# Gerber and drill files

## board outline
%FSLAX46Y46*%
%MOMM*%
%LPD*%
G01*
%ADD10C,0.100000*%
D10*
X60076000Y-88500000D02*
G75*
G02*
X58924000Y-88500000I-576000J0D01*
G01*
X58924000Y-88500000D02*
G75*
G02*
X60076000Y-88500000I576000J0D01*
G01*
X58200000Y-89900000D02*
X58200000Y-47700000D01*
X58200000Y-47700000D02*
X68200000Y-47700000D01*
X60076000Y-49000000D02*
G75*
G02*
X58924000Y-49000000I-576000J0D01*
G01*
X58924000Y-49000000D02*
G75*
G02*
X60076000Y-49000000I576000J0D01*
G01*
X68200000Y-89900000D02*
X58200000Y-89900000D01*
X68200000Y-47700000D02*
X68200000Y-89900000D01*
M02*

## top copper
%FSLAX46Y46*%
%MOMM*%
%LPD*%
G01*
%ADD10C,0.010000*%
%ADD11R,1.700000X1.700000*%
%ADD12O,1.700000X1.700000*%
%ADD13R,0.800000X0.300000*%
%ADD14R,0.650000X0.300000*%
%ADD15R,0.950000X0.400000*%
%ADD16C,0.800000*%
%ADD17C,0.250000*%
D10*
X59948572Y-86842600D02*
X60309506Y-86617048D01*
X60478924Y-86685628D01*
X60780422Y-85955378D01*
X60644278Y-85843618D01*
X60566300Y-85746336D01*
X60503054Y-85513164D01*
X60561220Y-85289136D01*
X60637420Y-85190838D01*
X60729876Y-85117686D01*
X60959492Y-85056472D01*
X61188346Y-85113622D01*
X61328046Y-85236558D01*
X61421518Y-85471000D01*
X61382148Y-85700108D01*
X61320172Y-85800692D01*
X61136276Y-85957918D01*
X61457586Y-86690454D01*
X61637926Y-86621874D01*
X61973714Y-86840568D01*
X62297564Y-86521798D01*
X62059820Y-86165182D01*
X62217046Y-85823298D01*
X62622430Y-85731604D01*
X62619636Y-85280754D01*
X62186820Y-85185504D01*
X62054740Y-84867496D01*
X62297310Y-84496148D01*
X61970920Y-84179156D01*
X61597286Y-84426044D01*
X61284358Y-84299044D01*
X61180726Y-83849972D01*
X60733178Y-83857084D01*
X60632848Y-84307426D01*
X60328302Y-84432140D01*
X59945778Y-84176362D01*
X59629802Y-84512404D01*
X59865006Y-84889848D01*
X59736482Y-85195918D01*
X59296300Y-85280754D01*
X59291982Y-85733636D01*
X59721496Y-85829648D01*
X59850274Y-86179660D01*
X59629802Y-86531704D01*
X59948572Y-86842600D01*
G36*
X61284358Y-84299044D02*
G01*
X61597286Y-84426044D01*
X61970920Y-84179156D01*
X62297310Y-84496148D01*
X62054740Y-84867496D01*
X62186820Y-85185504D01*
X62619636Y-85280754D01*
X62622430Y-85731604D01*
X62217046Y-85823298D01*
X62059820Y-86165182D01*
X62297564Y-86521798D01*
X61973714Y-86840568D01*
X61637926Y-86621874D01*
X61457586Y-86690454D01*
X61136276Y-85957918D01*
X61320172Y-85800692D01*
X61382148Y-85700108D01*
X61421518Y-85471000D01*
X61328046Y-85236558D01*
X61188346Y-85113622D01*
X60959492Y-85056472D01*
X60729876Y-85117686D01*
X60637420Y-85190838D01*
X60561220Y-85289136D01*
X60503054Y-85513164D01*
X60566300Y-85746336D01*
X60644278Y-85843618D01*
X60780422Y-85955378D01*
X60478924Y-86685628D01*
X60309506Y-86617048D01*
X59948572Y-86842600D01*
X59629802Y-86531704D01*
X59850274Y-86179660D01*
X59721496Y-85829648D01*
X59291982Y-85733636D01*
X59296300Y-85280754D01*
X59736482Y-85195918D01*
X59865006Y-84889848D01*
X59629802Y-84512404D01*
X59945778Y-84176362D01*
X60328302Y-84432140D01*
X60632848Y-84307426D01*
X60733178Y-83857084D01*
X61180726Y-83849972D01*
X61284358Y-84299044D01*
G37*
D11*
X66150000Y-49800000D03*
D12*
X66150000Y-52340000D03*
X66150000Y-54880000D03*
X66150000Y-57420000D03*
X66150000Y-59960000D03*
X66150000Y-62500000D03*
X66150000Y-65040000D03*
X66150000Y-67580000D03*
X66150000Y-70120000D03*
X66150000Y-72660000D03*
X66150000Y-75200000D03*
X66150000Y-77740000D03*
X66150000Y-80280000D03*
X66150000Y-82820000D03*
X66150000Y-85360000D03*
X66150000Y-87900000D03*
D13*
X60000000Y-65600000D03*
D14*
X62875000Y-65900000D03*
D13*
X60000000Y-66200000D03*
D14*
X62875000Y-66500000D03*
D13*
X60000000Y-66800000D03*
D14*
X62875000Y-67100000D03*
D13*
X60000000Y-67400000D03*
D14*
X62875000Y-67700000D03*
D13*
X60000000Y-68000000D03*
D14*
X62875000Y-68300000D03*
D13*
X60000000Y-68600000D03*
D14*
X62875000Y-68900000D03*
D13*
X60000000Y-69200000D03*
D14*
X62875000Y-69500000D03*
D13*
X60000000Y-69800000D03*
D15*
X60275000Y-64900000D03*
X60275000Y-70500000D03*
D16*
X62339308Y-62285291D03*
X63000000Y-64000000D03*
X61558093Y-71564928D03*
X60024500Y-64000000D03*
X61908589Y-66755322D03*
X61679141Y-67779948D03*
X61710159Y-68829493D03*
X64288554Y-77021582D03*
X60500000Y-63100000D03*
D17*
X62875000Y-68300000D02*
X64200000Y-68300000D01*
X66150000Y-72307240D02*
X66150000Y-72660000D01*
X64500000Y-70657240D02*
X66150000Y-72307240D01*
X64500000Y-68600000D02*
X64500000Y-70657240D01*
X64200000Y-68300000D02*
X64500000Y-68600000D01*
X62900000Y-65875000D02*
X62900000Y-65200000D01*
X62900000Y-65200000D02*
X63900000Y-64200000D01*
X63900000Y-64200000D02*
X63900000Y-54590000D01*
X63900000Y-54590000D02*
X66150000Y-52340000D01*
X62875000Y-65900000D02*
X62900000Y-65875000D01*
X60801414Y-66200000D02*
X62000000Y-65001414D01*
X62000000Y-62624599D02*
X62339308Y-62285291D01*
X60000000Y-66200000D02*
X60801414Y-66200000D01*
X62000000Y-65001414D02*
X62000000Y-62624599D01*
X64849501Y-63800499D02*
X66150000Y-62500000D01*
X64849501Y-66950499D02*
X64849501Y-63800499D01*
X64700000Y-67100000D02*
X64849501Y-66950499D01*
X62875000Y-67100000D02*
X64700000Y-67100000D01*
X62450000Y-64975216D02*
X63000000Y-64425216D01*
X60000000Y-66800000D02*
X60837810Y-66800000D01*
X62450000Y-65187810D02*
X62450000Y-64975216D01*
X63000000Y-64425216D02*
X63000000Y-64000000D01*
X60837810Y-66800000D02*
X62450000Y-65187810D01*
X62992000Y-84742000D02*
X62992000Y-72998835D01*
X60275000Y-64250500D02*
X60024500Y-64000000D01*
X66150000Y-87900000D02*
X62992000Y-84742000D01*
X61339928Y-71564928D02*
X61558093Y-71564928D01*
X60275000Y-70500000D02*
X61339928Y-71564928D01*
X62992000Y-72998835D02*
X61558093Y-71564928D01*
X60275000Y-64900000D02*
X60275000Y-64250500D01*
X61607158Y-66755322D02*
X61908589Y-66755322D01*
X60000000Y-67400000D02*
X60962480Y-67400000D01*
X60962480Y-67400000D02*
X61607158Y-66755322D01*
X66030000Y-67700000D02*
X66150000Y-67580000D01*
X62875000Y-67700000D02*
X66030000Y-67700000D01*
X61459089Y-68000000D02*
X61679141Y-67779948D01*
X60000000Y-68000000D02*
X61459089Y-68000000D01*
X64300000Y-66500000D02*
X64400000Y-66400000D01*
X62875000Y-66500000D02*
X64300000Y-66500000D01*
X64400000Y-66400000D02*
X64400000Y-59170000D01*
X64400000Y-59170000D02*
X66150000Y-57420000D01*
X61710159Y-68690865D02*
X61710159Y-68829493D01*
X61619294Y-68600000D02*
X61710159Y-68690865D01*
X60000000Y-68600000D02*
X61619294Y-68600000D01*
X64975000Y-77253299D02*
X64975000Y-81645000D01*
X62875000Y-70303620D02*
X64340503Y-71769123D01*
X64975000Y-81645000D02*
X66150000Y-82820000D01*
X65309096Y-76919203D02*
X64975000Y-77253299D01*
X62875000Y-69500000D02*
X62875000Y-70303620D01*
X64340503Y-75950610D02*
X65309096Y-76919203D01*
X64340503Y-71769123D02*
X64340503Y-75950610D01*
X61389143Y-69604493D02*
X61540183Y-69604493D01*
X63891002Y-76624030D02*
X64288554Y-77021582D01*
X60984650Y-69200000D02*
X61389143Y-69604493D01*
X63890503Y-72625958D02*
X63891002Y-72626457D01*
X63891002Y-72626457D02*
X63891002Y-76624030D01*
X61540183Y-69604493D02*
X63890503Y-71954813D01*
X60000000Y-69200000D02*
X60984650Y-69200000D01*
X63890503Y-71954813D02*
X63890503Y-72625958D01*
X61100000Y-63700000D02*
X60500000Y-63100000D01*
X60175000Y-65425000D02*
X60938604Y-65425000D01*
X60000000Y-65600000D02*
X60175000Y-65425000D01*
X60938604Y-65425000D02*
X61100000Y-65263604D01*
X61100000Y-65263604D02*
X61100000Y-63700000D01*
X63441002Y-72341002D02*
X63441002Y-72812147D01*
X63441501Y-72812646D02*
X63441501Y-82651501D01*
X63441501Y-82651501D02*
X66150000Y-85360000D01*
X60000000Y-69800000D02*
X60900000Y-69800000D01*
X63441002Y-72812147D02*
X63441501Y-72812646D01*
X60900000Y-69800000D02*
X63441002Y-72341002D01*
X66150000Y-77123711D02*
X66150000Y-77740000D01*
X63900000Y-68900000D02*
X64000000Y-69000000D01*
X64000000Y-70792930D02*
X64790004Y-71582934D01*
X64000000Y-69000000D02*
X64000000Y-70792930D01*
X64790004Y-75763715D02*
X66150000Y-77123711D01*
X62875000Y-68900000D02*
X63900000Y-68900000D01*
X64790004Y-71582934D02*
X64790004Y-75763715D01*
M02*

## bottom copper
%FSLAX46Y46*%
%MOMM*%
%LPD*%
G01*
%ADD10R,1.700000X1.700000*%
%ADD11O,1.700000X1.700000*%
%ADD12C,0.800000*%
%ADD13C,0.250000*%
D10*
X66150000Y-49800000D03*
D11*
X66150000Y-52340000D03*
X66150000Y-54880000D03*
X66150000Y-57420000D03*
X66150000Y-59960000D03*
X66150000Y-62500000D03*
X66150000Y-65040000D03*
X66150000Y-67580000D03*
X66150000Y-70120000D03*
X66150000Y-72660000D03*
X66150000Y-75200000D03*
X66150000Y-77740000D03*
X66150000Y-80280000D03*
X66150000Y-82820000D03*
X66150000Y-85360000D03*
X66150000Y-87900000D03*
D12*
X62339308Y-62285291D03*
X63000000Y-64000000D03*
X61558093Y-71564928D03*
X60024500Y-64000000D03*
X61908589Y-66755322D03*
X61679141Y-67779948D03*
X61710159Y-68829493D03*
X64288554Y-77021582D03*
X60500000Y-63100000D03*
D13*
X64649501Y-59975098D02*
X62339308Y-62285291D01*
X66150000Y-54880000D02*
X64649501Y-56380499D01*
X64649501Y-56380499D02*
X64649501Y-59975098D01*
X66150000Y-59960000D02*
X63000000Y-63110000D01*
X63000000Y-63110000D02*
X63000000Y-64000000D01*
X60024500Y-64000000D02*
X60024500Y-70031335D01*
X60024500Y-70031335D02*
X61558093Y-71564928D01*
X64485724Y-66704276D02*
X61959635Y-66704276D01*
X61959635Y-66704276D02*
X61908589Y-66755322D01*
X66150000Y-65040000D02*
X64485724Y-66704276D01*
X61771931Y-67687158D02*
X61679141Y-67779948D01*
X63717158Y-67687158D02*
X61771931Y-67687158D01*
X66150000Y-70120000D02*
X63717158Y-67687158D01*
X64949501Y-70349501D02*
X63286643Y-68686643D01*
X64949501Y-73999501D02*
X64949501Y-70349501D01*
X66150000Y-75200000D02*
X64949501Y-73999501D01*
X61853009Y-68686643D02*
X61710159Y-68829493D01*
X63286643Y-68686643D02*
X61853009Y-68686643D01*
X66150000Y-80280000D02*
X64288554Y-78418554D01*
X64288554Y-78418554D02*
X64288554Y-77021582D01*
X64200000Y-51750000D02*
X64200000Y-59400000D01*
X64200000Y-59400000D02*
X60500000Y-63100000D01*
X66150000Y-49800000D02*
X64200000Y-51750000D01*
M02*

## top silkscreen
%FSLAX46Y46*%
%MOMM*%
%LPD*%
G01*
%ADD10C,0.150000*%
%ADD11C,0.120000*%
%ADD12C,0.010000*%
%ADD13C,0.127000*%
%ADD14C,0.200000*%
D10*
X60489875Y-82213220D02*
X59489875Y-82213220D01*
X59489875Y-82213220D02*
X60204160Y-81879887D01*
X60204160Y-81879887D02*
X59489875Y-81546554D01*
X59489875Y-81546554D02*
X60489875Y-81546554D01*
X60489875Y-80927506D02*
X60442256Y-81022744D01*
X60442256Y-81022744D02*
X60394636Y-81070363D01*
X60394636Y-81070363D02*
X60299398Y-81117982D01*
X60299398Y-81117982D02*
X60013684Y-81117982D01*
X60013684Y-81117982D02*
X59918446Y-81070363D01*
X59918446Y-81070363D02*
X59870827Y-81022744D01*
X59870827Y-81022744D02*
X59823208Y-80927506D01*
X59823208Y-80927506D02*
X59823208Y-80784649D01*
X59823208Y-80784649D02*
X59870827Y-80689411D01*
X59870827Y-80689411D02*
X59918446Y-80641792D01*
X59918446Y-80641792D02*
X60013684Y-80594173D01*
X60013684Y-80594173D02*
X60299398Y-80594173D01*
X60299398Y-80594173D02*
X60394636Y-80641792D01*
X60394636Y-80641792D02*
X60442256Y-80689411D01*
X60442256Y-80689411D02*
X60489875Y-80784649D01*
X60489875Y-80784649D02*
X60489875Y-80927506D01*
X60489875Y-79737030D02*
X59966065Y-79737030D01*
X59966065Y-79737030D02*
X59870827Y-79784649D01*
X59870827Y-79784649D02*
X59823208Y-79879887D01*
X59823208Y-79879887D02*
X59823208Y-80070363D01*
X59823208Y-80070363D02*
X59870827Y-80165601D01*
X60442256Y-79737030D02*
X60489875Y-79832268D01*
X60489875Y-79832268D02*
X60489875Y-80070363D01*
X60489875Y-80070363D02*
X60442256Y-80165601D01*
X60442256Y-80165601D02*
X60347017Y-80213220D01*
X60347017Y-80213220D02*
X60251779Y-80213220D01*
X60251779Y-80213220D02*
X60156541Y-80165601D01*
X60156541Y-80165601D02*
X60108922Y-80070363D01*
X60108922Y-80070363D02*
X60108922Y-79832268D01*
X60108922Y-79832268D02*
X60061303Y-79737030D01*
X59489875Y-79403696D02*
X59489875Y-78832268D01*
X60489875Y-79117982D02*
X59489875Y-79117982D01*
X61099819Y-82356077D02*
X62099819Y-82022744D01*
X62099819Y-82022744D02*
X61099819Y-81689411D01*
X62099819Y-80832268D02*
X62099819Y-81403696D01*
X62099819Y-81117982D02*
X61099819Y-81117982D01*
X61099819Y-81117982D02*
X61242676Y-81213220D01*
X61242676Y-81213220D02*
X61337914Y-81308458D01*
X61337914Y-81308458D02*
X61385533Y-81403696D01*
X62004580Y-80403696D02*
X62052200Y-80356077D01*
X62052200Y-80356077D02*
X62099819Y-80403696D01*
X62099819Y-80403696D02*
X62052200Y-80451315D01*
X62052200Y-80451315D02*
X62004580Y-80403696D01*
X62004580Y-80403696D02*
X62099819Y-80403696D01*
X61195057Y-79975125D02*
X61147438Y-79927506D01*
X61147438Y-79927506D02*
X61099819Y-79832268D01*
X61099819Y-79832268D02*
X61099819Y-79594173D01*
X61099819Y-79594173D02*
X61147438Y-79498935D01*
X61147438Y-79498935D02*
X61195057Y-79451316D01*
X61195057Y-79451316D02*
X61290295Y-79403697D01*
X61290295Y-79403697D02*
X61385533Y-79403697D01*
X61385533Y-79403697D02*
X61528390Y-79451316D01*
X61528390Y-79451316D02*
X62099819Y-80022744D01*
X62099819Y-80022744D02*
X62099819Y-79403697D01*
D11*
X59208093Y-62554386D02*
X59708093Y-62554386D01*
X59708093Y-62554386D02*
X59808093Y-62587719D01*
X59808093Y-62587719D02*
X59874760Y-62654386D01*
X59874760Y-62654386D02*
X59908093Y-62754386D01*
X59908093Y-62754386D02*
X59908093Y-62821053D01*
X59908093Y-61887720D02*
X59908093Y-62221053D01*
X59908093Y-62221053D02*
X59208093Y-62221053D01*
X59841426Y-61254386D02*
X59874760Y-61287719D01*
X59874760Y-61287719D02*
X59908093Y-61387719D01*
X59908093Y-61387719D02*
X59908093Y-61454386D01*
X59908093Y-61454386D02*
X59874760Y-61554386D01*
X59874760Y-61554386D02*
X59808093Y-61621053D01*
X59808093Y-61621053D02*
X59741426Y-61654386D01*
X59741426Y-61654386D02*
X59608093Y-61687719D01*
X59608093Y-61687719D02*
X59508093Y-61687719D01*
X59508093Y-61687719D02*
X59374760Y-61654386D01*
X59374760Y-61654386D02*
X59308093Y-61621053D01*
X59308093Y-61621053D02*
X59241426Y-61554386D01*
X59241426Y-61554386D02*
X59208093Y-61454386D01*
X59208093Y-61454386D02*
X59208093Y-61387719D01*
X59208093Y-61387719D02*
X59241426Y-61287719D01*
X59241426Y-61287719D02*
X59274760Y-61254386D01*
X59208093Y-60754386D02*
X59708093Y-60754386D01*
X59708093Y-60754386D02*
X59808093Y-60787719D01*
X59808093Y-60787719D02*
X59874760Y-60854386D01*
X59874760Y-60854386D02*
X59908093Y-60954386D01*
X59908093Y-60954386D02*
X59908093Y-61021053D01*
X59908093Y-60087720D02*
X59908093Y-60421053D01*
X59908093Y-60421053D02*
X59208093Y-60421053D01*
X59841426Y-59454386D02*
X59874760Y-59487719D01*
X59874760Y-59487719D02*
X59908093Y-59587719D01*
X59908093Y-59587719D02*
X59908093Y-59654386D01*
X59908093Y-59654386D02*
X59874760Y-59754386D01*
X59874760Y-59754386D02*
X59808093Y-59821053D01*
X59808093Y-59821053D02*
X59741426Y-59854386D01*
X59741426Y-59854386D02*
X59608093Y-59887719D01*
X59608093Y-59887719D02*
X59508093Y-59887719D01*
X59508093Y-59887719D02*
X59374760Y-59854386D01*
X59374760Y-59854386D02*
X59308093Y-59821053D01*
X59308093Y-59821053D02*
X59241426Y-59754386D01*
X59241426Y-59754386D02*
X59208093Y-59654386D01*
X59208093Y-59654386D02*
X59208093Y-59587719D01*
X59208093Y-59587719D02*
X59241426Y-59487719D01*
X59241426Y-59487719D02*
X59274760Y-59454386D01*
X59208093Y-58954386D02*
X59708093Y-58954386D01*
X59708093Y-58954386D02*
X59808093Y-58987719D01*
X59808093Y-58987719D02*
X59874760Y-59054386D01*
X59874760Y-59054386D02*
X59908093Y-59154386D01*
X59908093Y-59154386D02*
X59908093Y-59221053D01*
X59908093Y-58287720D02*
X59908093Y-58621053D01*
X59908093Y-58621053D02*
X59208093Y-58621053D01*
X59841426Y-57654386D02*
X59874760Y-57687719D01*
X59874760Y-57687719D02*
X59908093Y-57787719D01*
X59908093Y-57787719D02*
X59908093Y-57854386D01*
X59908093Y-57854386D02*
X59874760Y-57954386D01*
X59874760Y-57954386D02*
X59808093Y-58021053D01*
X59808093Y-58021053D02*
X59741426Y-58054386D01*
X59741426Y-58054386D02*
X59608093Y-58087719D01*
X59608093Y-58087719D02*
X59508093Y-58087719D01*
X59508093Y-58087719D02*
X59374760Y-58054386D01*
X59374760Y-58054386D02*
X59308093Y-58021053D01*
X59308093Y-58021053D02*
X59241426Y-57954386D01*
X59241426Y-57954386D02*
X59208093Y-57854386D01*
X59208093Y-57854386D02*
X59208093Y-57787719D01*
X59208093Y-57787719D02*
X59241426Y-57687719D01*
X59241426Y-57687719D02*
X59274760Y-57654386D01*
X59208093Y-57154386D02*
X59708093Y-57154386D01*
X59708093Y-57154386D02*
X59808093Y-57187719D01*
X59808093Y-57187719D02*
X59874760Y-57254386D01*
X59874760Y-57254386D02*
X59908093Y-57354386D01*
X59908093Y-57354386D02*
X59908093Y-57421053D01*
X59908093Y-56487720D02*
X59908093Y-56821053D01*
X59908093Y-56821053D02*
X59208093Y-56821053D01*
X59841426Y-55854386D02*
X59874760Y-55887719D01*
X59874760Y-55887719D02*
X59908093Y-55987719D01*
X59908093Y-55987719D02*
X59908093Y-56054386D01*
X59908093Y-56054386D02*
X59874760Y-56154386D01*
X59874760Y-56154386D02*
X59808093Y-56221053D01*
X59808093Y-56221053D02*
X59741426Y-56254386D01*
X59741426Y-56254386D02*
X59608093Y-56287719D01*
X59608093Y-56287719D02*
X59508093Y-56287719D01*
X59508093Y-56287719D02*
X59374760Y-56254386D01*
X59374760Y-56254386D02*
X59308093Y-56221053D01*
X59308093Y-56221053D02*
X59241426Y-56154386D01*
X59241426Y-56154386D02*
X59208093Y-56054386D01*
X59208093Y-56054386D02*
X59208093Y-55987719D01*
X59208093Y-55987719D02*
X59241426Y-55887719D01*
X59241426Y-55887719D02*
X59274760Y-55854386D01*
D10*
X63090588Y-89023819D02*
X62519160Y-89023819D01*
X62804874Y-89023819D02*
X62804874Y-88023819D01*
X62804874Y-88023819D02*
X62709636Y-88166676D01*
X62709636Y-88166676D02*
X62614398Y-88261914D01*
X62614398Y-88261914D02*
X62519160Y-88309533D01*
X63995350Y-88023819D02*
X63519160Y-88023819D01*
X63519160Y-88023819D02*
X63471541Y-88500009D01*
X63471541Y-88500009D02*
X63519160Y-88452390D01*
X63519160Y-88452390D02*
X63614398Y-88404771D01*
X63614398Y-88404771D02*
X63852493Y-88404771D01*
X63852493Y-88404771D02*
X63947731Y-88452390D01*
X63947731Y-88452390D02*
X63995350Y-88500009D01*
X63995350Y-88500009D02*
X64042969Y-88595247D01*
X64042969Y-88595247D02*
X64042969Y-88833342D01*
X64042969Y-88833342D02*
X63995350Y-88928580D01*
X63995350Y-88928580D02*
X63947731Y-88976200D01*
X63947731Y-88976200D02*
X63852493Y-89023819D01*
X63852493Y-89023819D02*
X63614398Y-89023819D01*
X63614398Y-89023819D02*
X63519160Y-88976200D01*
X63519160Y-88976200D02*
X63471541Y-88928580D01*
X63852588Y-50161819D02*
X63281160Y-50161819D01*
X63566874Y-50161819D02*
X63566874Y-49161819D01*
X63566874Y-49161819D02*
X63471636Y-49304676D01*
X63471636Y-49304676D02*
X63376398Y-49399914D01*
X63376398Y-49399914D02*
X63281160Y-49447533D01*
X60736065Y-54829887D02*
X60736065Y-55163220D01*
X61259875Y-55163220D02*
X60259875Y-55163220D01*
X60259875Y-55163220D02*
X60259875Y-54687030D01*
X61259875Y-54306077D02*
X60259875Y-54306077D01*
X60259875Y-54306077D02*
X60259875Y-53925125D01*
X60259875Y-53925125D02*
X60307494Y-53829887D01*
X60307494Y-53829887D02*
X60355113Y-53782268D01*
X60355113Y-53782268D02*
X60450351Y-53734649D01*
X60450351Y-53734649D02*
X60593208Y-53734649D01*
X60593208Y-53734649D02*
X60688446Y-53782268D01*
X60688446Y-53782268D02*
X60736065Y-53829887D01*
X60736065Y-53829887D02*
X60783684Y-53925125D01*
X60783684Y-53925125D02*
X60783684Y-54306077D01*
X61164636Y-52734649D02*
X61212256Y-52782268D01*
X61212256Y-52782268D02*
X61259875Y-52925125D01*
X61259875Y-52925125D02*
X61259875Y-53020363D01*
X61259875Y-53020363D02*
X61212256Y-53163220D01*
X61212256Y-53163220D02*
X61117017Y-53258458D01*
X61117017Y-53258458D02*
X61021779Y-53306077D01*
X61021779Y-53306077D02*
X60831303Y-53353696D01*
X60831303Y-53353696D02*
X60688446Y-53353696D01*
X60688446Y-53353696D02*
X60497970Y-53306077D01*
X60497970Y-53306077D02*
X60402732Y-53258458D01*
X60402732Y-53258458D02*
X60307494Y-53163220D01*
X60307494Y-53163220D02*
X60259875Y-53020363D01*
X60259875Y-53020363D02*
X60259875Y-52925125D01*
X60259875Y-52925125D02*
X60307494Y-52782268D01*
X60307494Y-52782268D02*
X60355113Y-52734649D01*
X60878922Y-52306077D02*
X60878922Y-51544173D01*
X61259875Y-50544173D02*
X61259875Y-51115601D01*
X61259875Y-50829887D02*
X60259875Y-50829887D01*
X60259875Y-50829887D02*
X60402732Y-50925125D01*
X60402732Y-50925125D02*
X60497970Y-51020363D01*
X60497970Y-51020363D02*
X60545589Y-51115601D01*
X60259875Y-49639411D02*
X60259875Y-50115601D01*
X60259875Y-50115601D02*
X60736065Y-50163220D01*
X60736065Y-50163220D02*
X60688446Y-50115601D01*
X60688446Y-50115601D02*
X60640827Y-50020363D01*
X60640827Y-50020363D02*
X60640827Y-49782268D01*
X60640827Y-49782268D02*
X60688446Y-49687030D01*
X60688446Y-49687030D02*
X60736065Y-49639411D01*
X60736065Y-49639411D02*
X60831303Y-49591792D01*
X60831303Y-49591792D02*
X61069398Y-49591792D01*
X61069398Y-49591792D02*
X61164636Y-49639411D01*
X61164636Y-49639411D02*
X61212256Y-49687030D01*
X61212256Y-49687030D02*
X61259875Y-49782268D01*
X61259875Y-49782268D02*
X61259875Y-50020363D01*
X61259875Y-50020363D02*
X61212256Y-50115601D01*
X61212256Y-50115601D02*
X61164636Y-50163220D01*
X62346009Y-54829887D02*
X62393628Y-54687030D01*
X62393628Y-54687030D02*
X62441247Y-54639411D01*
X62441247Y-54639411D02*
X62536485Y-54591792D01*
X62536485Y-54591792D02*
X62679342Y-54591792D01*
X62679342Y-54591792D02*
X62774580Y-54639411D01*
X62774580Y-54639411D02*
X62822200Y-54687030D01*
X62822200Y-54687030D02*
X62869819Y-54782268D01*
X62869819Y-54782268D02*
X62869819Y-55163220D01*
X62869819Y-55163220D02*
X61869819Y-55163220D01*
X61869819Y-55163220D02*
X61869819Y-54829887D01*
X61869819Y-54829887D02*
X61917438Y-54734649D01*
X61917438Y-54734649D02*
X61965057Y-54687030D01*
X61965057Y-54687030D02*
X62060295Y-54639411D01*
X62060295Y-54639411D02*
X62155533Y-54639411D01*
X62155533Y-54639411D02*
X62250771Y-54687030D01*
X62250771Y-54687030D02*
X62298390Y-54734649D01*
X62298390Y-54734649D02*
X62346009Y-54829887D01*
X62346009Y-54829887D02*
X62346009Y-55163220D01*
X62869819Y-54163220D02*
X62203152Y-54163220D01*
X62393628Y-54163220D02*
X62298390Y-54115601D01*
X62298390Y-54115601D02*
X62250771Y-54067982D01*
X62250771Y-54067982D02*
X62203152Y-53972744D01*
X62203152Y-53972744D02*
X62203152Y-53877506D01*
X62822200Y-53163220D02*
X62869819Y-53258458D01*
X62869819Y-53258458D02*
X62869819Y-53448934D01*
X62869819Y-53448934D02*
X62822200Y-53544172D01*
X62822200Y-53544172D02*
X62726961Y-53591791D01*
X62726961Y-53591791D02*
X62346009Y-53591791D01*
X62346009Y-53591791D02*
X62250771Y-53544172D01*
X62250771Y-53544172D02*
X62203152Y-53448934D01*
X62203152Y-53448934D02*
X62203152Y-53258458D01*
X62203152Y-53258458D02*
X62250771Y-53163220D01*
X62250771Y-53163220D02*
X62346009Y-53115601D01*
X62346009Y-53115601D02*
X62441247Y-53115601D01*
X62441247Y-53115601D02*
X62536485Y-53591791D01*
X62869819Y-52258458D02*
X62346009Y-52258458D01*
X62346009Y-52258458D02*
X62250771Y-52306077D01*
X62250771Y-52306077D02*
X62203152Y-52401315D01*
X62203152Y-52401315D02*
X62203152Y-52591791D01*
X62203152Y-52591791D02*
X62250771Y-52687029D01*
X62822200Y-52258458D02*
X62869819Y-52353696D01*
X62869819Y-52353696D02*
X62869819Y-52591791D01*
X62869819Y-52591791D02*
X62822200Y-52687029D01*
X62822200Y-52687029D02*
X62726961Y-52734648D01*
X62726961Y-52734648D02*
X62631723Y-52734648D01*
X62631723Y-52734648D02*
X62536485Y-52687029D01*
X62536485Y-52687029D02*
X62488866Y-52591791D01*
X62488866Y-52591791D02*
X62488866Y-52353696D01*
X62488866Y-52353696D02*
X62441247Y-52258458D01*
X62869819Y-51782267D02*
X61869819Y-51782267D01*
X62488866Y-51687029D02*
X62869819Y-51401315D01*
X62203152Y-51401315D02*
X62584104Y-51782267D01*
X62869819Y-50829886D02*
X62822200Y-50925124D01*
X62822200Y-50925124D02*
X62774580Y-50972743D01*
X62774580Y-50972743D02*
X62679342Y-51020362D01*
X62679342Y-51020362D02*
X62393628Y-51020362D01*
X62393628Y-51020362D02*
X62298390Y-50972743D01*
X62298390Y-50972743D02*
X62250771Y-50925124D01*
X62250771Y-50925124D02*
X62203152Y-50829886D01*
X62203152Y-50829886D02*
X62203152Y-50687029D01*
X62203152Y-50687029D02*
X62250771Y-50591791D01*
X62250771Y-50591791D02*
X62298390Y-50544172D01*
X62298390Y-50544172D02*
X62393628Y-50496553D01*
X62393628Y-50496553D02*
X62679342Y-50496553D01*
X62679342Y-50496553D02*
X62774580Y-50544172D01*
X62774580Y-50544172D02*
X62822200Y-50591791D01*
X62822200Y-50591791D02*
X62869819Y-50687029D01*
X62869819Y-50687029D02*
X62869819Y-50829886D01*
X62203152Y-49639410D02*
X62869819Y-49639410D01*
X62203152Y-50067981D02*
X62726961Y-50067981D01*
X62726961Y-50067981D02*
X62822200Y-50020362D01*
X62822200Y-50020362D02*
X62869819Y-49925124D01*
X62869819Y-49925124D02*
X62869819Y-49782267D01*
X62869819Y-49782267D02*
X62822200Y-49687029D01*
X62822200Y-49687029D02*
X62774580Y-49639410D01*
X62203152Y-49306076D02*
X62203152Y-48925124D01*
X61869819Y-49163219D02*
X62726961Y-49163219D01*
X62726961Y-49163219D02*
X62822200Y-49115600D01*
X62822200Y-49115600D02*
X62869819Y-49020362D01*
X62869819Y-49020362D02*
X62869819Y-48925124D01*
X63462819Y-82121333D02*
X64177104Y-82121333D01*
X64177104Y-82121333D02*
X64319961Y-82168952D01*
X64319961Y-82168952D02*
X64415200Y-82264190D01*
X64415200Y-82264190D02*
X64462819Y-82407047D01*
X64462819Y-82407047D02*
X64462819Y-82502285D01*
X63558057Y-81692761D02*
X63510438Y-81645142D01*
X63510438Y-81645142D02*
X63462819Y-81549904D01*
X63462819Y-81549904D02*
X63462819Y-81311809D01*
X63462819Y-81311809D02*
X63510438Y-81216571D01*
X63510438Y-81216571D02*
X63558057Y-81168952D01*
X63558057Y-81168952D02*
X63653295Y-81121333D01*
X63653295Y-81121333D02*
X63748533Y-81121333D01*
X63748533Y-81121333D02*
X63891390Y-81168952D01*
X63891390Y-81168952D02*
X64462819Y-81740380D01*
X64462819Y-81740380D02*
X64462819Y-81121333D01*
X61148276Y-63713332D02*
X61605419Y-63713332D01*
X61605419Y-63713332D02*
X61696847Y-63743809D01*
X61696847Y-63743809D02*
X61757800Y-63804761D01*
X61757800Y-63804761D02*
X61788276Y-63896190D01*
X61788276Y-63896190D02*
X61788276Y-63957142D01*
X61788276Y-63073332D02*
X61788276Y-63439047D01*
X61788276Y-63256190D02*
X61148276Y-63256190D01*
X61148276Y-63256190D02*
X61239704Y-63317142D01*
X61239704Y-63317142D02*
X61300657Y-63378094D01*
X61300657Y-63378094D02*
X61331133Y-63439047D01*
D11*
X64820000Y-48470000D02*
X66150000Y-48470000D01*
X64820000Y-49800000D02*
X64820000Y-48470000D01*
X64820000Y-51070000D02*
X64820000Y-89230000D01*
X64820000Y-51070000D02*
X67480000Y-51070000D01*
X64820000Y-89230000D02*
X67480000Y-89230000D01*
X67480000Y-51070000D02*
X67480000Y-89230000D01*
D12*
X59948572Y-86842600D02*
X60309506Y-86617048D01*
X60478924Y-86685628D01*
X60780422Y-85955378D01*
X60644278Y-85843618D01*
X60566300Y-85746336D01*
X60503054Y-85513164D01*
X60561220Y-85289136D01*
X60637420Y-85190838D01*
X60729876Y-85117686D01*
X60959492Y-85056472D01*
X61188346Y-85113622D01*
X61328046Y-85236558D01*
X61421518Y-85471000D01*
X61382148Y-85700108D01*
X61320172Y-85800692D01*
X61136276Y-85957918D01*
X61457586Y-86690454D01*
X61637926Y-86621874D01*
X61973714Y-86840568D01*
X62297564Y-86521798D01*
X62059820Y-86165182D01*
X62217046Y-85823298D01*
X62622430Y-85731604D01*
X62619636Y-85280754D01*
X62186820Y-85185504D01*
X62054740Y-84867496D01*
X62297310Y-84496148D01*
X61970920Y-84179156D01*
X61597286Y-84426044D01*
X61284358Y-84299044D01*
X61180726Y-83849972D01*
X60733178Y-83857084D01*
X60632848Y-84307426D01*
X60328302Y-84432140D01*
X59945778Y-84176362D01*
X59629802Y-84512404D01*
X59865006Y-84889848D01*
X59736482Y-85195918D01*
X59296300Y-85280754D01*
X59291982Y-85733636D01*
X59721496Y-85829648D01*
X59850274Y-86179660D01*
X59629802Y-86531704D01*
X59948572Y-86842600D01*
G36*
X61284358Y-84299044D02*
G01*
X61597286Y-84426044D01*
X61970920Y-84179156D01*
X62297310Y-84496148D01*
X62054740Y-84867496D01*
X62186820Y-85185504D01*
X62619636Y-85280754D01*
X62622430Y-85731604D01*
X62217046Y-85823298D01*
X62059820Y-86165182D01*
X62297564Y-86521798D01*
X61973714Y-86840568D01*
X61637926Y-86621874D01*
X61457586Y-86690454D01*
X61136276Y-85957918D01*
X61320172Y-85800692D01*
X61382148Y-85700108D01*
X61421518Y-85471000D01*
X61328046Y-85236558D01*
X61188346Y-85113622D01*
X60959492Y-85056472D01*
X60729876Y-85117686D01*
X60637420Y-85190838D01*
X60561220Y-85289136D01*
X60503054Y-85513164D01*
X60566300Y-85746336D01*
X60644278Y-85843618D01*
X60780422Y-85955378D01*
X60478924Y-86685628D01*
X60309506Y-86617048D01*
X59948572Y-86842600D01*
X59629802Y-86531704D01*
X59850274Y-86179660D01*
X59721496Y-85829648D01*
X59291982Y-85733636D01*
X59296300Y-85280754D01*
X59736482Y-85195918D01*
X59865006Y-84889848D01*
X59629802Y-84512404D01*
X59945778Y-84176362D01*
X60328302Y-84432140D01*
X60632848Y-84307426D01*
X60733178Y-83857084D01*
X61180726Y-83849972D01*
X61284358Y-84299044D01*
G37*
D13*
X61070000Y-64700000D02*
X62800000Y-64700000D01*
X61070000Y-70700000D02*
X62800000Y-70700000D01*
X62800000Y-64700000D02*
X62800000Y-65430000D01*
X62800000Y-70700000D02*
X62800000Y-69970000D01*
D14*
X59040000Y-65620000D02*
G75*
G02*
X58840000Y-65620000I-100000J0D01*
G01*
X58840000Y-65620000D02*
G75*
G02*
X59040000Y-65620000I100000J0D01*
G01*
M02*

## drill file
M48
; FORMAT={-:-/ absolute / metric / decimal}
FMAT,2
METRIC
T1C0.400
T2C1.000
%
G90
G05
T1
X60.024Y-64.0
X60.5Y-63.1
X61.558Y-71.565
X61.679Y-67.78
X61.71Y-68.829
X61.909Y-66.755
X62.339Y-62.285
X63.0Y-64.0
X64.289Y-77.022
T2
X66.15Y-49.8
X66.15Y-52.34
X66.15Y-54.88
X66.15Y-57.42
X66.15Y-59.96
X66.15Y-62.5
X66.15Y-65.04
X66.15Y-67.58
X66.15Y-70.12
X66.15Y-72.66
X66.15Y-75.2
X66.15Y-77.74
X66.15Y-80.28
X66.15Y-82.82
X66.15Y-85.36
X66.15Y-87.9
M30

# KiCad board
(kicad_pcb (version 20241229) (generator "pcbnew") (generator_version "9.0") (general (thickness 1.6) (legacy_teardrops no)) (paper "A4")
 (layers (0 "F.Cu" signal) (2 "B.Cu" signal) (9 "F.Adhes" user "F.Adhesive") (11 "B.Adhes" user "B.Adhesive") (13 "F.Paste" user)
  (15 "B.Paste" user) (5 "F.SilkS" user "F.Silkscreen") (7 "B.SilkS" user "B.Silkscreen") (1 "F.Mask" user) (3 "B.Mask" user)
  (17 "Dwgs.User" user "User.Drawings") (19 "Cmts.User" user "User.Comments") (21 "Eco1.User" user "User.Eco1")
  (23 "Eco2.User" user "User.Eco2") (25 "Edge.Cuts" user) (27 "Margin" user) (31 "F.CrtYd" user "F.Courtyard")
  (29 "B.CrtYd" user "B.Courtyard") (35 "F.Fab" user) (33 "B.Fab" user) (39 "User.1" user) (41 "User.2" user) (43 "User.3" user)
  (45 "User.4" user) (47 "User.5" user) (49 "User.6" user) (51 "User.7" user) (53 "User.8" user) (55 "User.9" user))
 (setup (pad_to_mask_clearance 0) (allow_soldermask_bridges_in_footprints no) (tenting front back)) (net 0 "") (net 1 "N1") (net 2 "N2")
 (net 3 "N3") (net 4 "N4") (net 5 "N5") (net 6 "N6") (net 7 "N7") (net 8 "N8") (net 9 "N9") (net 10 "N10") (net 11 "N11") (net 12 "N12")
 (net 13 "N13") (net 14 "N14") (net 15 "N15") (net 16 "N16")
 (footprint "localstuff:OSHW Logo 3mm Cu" (layer "F.Cu") (at 60.96 85.344)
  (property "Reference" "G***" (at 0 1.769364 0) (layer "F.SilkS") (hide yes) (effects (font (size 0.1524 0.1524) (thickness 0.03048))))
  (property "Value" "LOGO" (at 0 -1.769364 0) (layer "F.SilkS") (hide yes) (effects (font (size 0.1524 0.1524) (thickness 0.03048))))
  (fp_poly
   (pts (xy -1.011428 1.4986) (xy -0.650494 1.273048) (xy -0.481076 1.341628) (xy -0.179578 0.611378) (xy -0.315722 0.499618)
    (xy -0.3937 0.402336) (xy -0.456946 0.169164) (xy -0.39878 -0.054864) (xy -0.32258 -0.153162) (xy -0.230124 -0.226314)
    (xy -0.000508 -0.287528) (xy 0.228346 -0.230378) (xy 0.368046 -0.107442) (xy 0.461518 0.127) (xy 0.422148 0.356108)
    (xy 0.360172 0.456692) (xy 0.176276 0.613918) (xy 0.497586 1.346454) (xy 0.677926 1.277874) (xy 1.013714 1.496568)
    (xy 1.337564 1.177798) (xy 1.09982 0.821182) (xy 1.257046 0.479298) (xy 1.66243 0.387604) (xy 1.659636 -0.063246) (xy 1.22682 -0.158496)
    (xy 1.09474 -0.476504) (xy 1.33731 -0.847852) (xy 1.01092 -1.164844) (xy 0.637286 -0.917956) (xy 0.324358 -1.044956)
    (xy 0.220726 -1.494028) (xy -0.226822 -1.486916) (xy -0.327152 -1.036574) (xy -0.631698 -0.91186) (xy -1.014222 -1.167638)
    (xy -1.330198 -0.831596) (xy -1.094994 -0.454152) (xy -1.223518 -0.148082) (xy -1.6637 -0.063246) (xy -1.668018 0.389636)
    (xy -1.238504 0.485648) (xy -1.109726 0.83566) (xy -1.330198 1.187704) (xy -1.011428 1.4986))
   (stroke (width 0.01) (type solid)) (fill yes) (layer "F.Cu")))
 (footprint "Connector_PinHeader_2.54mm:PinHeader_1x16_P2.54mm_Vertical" (layer "F.Cu") (at 66.15 49.8)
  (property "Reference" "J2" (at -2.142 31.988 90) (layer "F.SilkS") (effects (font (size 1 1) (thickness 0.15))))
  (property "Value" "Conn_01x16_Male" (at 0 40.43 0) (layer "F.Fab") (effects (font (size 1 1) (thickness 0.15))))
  (fp_line (start -1.33 -1.33) (end 0 -1.33) (stroke (width 0.12) (type solid)) (layer "F.SilkS"))
  (fp_line (start -1.33 0) (end -1.33 -1.33) (stroke (width 0.12) (type solid)) (layer "F.SilkS"))
  (fp_line (start -1.33 1.27) (end -1.33 39.43) (stroke (width 0.12) (type solid)) (layer "F.SilkS"))
  (fp_line (start -1.33 1.27) (end 1.33 1.27) (stroke (width 0.12) (type solid)) (layer "F.SilkS"))
  (fp_line (start -1.33 39.43) (end 1.33 39.43) (stroke (width 0.12) (type solid)) (layer "F.SilkS"))
  (fp_line (start 1.33 1.27) (end 1.33 39.43) (stroke (width 0.12) (type solid)) (layer "F.SilkS"))
  (pad "1" thru_hole rect (at 0 0) (size 1.7 1.7) (drill 1) (layers "*.Cu" "*.Mask") (remove_unused_layers no) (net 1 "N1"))
  (pad "2" thru_hole oval (at 0 2.54) (size 1.7 1.7) (drill 1) (layers "*.Cu" "*.Mask") (remove_unused_layers no) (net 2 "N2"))
  (pad "3" thru_hole oval (at 0 5.08) (size 1.7 1.7) (drill 1) (layers "*.Cu" "*.Mask") (remove_unused_layers no) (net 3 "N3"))
  (pad "4" thru_hole oval (at 0 7.62) (size 1.7 1.7) (drill 1) (layers "*.Cu" "*.Mask") (remove_unused_layers no) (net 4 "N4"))
  (pad "5" thru_hole oval (at 0 10.16) (size 1.7 1.7) (drill 1) (layers "*.Cu" "*.Mask") (remove_unused_layers no) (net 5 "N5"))
  (pad "6" thru_hole oval (at 0 12.7) (size 1.7 1.7) (drill 1) (layers "*.Cu" "*.Mask") (remove_unused_layers no) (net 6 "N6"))
  (pad "7" thru_hole oval (at 0 15.24) (size 1.7 1.7) (drill 1) (layers "*.Cu" "*.Mask") (remove_unused_layers no) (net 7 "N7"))
  (pad "8" thru_hole oval (at 0 17.78) (size 1.7 1.7) (drill 1) (layers "*.Cu" "*.Mask") (remove_unused_layers no) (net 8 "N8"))
  (pad "9" thru_hole oval (at 0 20.32) (size 1.7 1.7) (drill 1) (layers "*.Cu" "*.Mask") (remove_unused_layers no) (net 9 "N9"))
  (pad "10" thru_hole oval (at 0 22.86) (size 1.7 1.7) (drill 1) (layers "*.Cu" "*.Mask") (remove_unused_layers no) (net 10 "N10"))
  (pad "11" thru_hole oval (at 0 25.4) (size 1.7 1.7) (drill 1) (layers "*.Cu" "*.Mask") (remove_unused_layers no) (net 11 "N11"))
  (pad "12" thru_hole oval (at 0 27.94) (size 1.7 1.7) (drill 1) (layers "*.Cu" "*.Mask") (remove_unused_layers no) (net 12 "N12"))
  (pad "13" thru_hole oval (at 0 30.48) (size 1.7 1.7) (drill 1) (layers "*.Cu" "*.Mask") (remove_unused_layers no) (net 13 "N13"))
  (pad "14" thru_hole oval (at 0 33.02) (size 1.7 1.7) (drill 1) (layers "*.Cu" "*.Mask") (remove_unused_layers no) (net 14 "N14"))
  (pad "15" thru_hole oval (at 0 35.56) (size 1.7 1.7) (drill 1) (layers "*.Cu" "*.Mask") (remove_unused_layers no) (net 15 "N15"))
  (pad "16" thru_hole oval (at 0 38.1) (size 1.7 1.7) (drill 1) (layers "*.Cu" "*.Mask") (remove_unused_layers no) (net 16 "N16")))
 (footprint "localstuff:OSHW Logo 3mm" (layer "F.Cu") (at 60.96 85.344)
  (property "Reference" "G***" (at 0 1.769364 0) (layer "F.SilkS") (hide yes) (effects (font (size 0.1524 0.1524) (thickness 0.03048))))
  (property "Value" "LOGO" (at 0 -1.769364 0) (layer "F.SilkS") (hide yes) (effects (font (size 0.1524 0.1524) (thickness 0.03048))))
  (fp_poly
   (pts (xy -1.011428 1.4986) (xy -0.650494 1.273048) (xy -0.481076 1.341628) (xy -0.179578 0.611378) (xy -0.315722 0.499618)
    (xy -0.3937 0.402336) (xy -0.456946 0.169164) (xy -0.39878 -0.054864) (xy -0.32258 -0.153162) (xy -0.230124 -0.226314)
    (xy -0.000508 -0.287528) (xy 0.228346 -0.230378) (xy 0.368046 -0.107442) (xy 0.461518 0.127) (xy 0.422148 0.356108)
    (xy 0.360172 0.456692) (xy 0.176276 0.613918) (xy 0.497586 1.346454) (xy 0.677926 1.277874) (xy 1.013714 1.496568)
    (xy 1.337564 1.177798) (xy 1.09982 0.821182) (xy 1.257046 0.479298) (xy 1.66243 0.387604) (xy 1.659636 -0.063246) (xy 1.22682 -0.158496)
    (xy 1.09474 -0.476504) (xy 1.33731 -0.847852) (xy 1.01092 -1.164844) (xy 0.637286 -0.917956) (xy 0.324358 -1.044956)
    (xy 0.220726 -1.494028) (xy -0.226822 -1.486916) (xy -0.327152 -1.036574) (xy -0.631698 -0.91186) (xy -1.014222 -1.167638)
    (xy -1.330198 -0.831596) (xy -1.094994 -0.454152) (xy -1.223518 -0.148082) (xy -1.6637 -0.063246) (xy -1.668018 0.389636)
    (xy -1.238504 0.485648) (xy -1.109726 0.83566) (xy -1.330198 1.187704) (xy -1.011428 1.4986))
   (stroke (width 0.01) (type solid)) (fill yes) (layer "F.SilkS")))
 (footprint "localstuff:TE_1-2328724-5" (layer "F.Cu") (at 61.4 67.7 -90)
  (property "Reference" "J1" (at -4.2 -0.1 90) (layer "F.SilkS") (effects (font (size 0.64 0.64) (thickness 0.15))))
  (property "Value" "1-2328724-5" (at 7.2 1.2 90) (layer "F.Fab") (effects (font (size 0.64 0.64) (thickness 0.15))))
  (fp_line (start -3 0.33) (end -3 -1.4) (stroke (width 0.127) (type solid)) (layer "F.SilkS"))
  (fp_line (start 3 0.33) (end 3 -1.4) (stroke (width 0.127) (type solid)) (layer "F.SilkS"))
  (fp_line (start -3 -1.4) (end -2.27 -1.4) (stroke (width 0.127) (type solid)) (layer "F.SilkS"))
  (fp_line (start 3 -1.4) (end 2.27 -1.4) (stroke (width 0.127) (type solid)) (layer "F.SilkS"))
  (fp_circle (center -2.08 2.46) (end -1.98 2.46) (stroke (width 0.2) (type solid)) (fill no) (layer "F.SilkS"))
  (pad "1" smd rect (at -2.1 1.4 90) (size 0.3 0.8) (layers "F.Cu" "F.Mask") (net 1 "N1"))
  (pad "2" smd rect (at -1.8 -1.475 90) (size 0.3 0.65) (layers "F.Cu" "F.Mask") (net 2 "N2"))
  (pad "3" smd rect (at -1.5 1.4 90) (size 0.3 0.8) (layers "F.Cu" "F.Mask") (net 3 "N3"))
  (pad "4" smd rect (at -1.2 -1.475 90) (size 0.3 0.65) (layers "F.Cu" "F.Mask") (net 4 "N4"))
  (pad "5" smd rect (at -0.9 1.4 90) (size 0.3 0.8) (layers "F.Cu" "F.Mask") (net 5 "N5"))
  (pad "6" smd rect (at -0.6 -1.475 90) (size 0.3 0.65) (layers "F.Cu" "F.Mask") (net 6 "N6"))
  (pad "7" smd rect (at -0.3 1.4 90) (size 0.3 0.8) (layers "F.Cu" "F.Mask") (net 7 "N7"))
  (pad "8" smd rect (at 0 -1.475 90) (size 0.3 0.65) (layers "F.Cu" "F.Mask") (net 8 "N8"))
  (pad "9" smd rect (at 0.3 1.4 90) (size 0.3 0.8) (layers "F.Cu" "F.Mask") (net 9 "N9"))
  (pad "10" smd rect (at 0.6 -1.475 90) (size 0.3 0.65) (layers "F.Cu" "F.Mask") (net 10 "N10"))
  (pad "11" smd rect (at 0.9 1.4 90) (size 0.3 0.8) (layers "F.Cu" "F.Mask") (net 11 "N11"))
  (pad "12" smd rect (at 1.2 -1.475 90) (size 0.3 0.65) (layers "F.Cu" "F.Mask") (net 12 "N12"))
  (pad "13" smd rect (at 1.5 1.4 90) (size 0.3 0.8) (layers "F.Cu" "F.Mask") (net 13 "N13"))
  (pad "14" smd rect (at 1.8 -1.475 90) (size 0.3 0.65) (layers "F.Cu" "F.Mask") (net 14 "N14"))
  (pad "15" smd rect (at 2.1 1.4 90) (size 0.3 0.8) (layers "F.Cu" "F.Mask") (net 15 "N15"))
  (pad "S1" smd rect (at -2.8 1.125 90) (size 0.4 0.95) (layers "F.Cu" "F.Mask") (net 16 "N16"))
  (pad "S2" smd rect (at 2.8 1.125 90) (size 0.4 0.95) (layers "F.Cu" "F.Mask") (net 16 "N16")))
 (gr_circle (center 59.5 88.5) (end 60.076 88.5) (stroke (width 0.1) (type solid)) (fill no) (layer "Edge.Cuts"))
 (gr_line (start 58.2 89.9) (end 58.2 47.7) (stroke (width 0.1) (type solid)) (layer "Edge.Cuts"))
 (gr_line (start 58.2 47.7) (end 68.2 47.7) (stroke (width 0.1) (type default)) (layer "Edge.Cuts"))
 (gr_circle (center 59.5 49) (end 60.076 49) (stroke (width 0.1) (type solid)) (fill no) (layer "Edge.Cuts"))
 (gr_line (start 68.2 89.9) (end 58.2 89.9) (stroke (width 0.1) (type default)) (layer "Edge.Cuts"))
 (gr_line (start 68.2 47.7) (end 68.2 89.9) (stroke (width 0.1) (type default)) (layer "Edge.Cuts"))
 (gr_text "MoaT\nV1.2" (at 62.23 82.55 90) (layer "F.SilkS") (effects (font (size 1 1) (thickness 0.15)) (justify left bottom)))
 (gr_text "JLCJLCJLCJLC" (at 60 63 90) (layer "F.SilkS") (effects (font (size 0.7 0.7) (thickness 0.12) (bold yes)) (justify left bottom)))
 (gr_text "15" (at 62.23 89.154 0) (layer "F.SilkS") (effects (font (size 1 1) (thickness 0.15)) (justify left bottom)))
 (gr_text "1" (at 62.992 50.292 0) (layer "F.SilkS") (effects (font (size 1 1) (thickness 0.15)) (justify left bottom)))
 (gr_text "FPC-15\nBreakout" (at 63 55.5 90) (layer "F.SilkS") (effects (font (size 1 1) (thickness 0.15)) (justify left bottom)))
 (segment (start 62.875 68.3) (end 64.2 68.3) (width 0.25) (layer "F.Cu") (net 10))
 (segment (start 66.15 72.30724) (end 66.15 72.66) (width 0.25) (layer "F.Cu") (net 10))
 (segment (start 64.5 70.65724) (end 66.15 72.30724) (width 0.25) (layer "F.Cu") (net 10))
 (segment (start 64.5 68.6) (end 64.5 70.65724) (width 0.25) (layer "F.Cu") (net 10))
 (segment (start 64.2 68.3) (end 64.5 68.6) (width 0.25) (layer "F.Cu") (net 10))
 (segment (start 62.9 65.875) (end 62.9 65.2) (width 0.25) (layer "F.Cu") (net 2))
 (segment (start 62.9 65.2) (end 63.9 64.2) (width 0.25) (layer "F.Cu") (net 2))
 (segment (start 63.9 64.2) (end 63.9 54.59) (width 0.25) (layer "F.Cu") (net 2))
 (segment (start 63.9 54.59) (end 66.15 52.34) (width 0.25) (layer "F.Cu") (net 2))
 (segment (start 62.875 65.9) (end 62.9 65.875) (width 0.25) (layer "F.Cu") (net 2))
 (segment (start 60.801414 66.2) (end 62 65.001414) (width 0.25) (layer "F.Cu") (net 3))
 (segment (start 62 62.624599) (end 62.339308 62.285291) (width 0.25) (layer "F.Cu") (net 3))
 (segment (start 60 66.2) (end 60.801414 66.2) (width 0.25) (layer "F.Cu") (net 3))
 (segment (start 62 65.001414) (end 62 62.624599) (width 0.25) (layer "F.Cu") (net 3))
 (via (at 62.339308 62.285291) (size 0.8) (drill 0.4) (layers "F.Cu" "B.Cu") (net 3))
 (segment (start 64.649501 59.975098) (end 62.339308 62.285291) (width 0.25) (layer "B.Cu") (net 3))
 (segment (start 66.15 54.88) (end 64.649501 56.380499) (width 0.25) (layer "B.Cu") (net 3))
 (segment (start 64.649501 56.380499) (end 64.649501 59.975098) (width 0.25) (layer "B.Cu") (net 3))
 (segment (start 64.849501 63.800499) (end 66.15 62.5) (width 0.25) (layer "F.Cu") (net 6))
 (segment (start 64.849501 66.950499) (end 64.849501 63.800499) (width 0.25) (layer "F.Cu") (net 6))
 (segment (start 64.7 67.1) (end 64.849501 66.950499) (width 0.25) (layer "F.Cu") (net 6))
 (segment (start 62.875 67.1) (end 64.7 67.1) (width 0.25) (layer "F.Cu") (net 6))
 (segment (start 62.45 64.975216) (end 63 64.425216) (width 0.25) (layer "F.Cu") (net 5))
 (segment (start 60 66.8) (end 60.83781 66.8) (width 0.25) (layer "F.Cu") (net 5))
 (segment (start 62.45 65.18781) (end 62.45 64.975216) (width 0.25) (layer "F.Cu") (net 5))
 (segment (start 63 64.425216) (end 63 64) (width 0.25) (layer "F.Cu") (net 5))
 (segment (start 60.83781 66.8) (end 62.45 65.18781) (width 0.25) (layer "F.Cu") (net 5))
 (via (at 63 64) (size 0.8) (drill 0.4) (layers "F.Cu" "B.Cu") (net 5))
 (segment (start 66.15 59.96) (end 63 63.11) (width 0.25) (layer "B.Cu") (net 5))
 (segment (start 63 63.11) (end 63 64) (width 0.25) (layer "B.Cu") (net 5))
 (segment (start 62.992 84.742) (end 62.992 72.998835) (width 0.25) (layer "F.Cu") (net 16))
 (segment (start 60.275 64.2505) (end 60.0245 64) (width 0.25) (layer "F.Cu") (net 16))
 (segment (start 66.15 87.9) (end 62.992 84.742) (width 0.25) (layer "F.Cu") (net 16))
 (segment (start 61.339928 71.564928) (end 61.558093 71.564928) (width 0.25) (layer "F.Cu") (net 16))
 (segment (start 60.275 70.5) (end 61.339928 71.564928) (width 0.25) (layer "F.Cu") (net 16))
 (segment (start 62.992 72.998835) (end 61.558093 71.564928) (width 0.25) (layer "F.Cu") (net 16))
 (segment (start 60.275 64.9) (end 60.275 64.2505) (width 0.25) (layer "F.Cu") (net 16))
 (via (at 61.558093 71.564928) (size 0.8) (drill 0.4) (layers "F.Cu" "B.Cu") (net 16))
 (via (at 60.0245 64) (size 0.8) (drill 0.4) (layers "F.Cu" "B.Cu") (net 16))
 (segment (start 60.0245 64) (end 60.0245 70.031335) (width 0.25) (layer "B.Cu") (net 16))
 (segment (start 60.0245 70.031335) (end 61.558093 71.564928) (width 0.25) (layer "B.Cu") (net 16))
 (segment (start 61.607158 66.755322) (end 61.908589 66.755322) (width 0.25) (layer "F.Cu") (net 7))
 (segment (start 60 67.4) (end 60.96248 67.4) (width 0.25) (layer "F.Cu") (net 7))
 (segment (start 60.96248 67.4) (end 61.607158 66.755322) (width 0.25) (layer "F.Cu") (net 7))
 (via (at 61.908589 66.755322) (size 0.8) (drill 0.4) (layers "F.Cu" "B.Cu") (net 7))
 (segment (start 64.485724 66.704276) (end 61.959635 66.704276) (width 0.25) (layer "B.Cu") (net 7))
 (segment (start 61.959635 66.704276) (end 61.908589 66.755322) (width 0.25) (layer "B.Cu") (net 7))
 (segment (start 66.15 65.04) (end 64.485724 66.704276) (width 0.25) (layer "B.Cu") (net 7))
 (segment (start 66.03 67.7) (end 66.15 67.58) (width 0.25) (layer "F.Cu") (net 8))
 (segment (start 62.875 67.7) (end 66.03 67.7) (width 0.25) (layer "F.Cu") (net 8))
 (segment (start 61.459089 68) (end 61.679141 67.779948) (width 0.25) (layer "F.Cu") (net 9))
 (segment (start 60 68) (end 61.459089 68) (width 0.25) (layer "F.Cu") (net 9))
 (via (at 61.679141 67.779948) (size 0.8) (drill 0.4) (layers "F.Cu" "B.Cu") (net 9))
 (segment (start 61.771931 67.687158) (end 61.679141 67.779948) (width 0.25) (layer "B.Cu") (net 9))
 (segment (start 63.717158 67.687158) (end 61.771931 67.687158) (width 0.25) (layer "B.Cu") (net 9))
 (segment (start 66.15 70.12) (end 63.717158 67.687158) (width 0.25) (layer "B.Cu") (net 9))
 (segment (start 64.3 66.5) (end 64.4 66.4) (width 0.25) (layer "F.Cu") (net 4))
 (segment (start 62.875 66.5) (end 64.3 66.5) (width 0.25) (layer "F.Cu") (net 4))
 (segment (start 64.4 66.4) (end 64.4 59.17) (width 0.25) (layer "F.Cu") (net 4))
 (segment (start 64.4 59.17) (end 66.15 57.42) (width 0.25) (layer "F.Cu") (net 4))
 (segment (start 61.710159 68.690865) (end 61.710159 68.829493) (width 0.25) (layer "F.Cu") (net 11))
 (segment (start 61.619294 68.6) (end 61.710159 68.690865) (width 0.25) (layer "F.Cu") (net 11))
 (segment (start 60 68.6) (end 61.619294 68.6) (width 0.25) (layer "F.Cu") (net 11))
 (via (at 61.710159 68.829493) (size 0.8) (drill 0.4) (layers "F.Cu" "B.Cu") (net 11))
 (segment (start 64.949501 70.349501) (end 63.286643 68.686643) (width 0.25) (layer "B.Cu") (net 11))
 (segment (start 64.949501 73.999501) (end 64.949501 70.349501) (width 0.25) (layer "B.Cu") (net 11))
 (segment (start 66.15 75.2) (end 64.949501 73.999501) (width 0.25) (layer "B.Cu") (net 11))
 (segment (start 61.853009 68.686643) (end 61.710159 68.829493) (width 0.25) (layer "B.Cu") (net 11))
 (segment (start 63.286643 68.686643) (end 61.853009 68.686643) (width 0.25) (layer "B.Cu") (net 11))
 (segment (start 64.975 77.253299) (end 64.975 81.645) (width 0.25) (layer "F.Cu") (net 14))
 (segment (start 62.875 70.30362) (end 64.340503 71.769123) (width 0.25) (layer "F.Cu") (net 14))
 (segment (start 64.975 81.645) (end 66.15 82.82) (width 0.25) (layer "F.Cu") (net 14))
 (segment (start 65.309096 76.919203) (end 64.975 77.253299) (width 0.25) (layer "F.Cu") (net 14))
 (segment (start 62.875 69.5) (end 62.875 70.30362) (width 0.25) (layer "F.Cu") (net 14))
 (segment (start 64.340503 75.95061) (end 65.309096 76.919203) (width 0.25) (layer "F.Cu") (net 14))
 (segment (start 64.340503 71.769123) (end 64.340503 75.95061) (width 0.25) (layer "F.Cu") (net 14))
 (segment (start 61.389143 69.604493) (end 61.540183 69.604493) (width 0.25) (layer "F.Cu") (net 13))
 (segment (start 63.891002 76.62403) (end 64.288554 77.021582) (width 0.25) (layer "F.Cu") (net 13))
 (segment (start 60.98465 69.2) (end 61.389143 69.604493) (width 0.25) (layer "F.Cu") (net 13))
 (segment (start 63.890503 72.625958) (end 63.891002 72.626457) (width 0.25) (layer "F.Cu") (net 13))
 (segment (start 63.891002 72.626457) (end 63.891002 76.62403) (width 0.25) (layer "F.Cu") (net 13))
 (segment (start 61.540183 69.604493) (end 63.890503 71.954813) (width 0.25) (layer "F.Cu") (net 13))
 (segment (start 60 69.2) (end 60.98465 69.2) (width 0.25) (layer "F.Cu") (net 13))
 (segment (start 63.890503 71.954813) (end 63.890503 72.625958) (width 0.25) (layer "F.Cu") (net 13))
 (via (at 64.288554 77.021582) (size 0.8) (drill 0.4) (layers "F.Cu" "B.Cu") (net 13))
 (segment (start 66.15 80.28) (end 64.288554 78.418554) (width 0.25) (layer "B.Cu") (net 13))
 (segment (start 64.288554 78.418554) (end 64.288554 77.021582) (width 0.25) (layer "B.Cu") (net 13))
 (segment (start 61.1 63.7) (end 60.5 63.1) (width 0.25) (layer "F.Cu") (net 1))
 (segment (start 60.175 65.425) (end 60.938604 65.425) (width 0.25) (layer "F.Cu") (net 1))
 (segment (start 60 65.6) (end 60.175 65.425) (width 0.25) (layer "F.Cu") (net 1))
 (segment (start 60.938604 65.425) (end 61.1 65.263604) (width 0.25) (layer "F.Cu") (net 1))
 (segment (start 61.1 65.263604) (end 61.1 63.7) (width 0.25) (layer "F.Cu") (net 1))
 (via (at 60.5 63.1) (size 0.8) (drill 0.4) (layers "F.Cu" "B.Cu") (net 1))
 (segment (start 64.2 51.75) (end 64.2 59.4) (width 0.25) (layer "B.Cu") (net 1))
 (segment (start 64.2 59.4) (end 60.5 63.1) (width 0.25) (layer "B.Cu") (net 1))
 (segment (start 66.15 49.8) (end 64.2 51.75) (width 0.25) (layer "B.Cu") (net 1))
 (segment (start 63.441002 72.341002) (end 63.441002 72.812147) (width 0.25) (layer "F.Cu") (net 15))
 (segment (start 63.441501 72.812646) (end 63.441501 82.651501) (width 0.25) (layer "F.Cu") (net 15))
 (segment (start 63.441501 82.651501) (end 66.15 85.36) (width 0.25) (layer "F.Cu") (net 15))
 (segment (start 60 69.8) (end 60.9 69.8) (width 0.25) (layer "F.Cu") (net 15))
 (segment (start 63.441002 72.812147) (end 63.441501 72.812646) (width 0.25) (layer "F.Cu") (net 15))
 (segment (start 60.9 69.8) (end 63.441002 72.341002) (width 0.25) (layer "F.Cu") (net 15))
 (segment (start 66.15 77.123711) (end 66.15 77.74) (width 0.25) (layer "F.Cu") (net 12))
 (segment (start 63.9 68.9) (end 64 69) (width 0.25) (layer "F.Cu") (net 12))
 (segment (start 64 70.79293) (end 64.790004 71.582934) (width 0.25) (layer "F.Cu") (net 12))
 (segment (start 64 69) (end 64 70.79293) (width 0.25) (layer "F.Cu") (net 12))
 (segment (start 64.790004 75.763715) (end 66.15 77.123711) (width 0.25) (layer "F.Cu") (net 12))
 (segment (start 62.875 68.9) (end 63.9 68.9) (width 0.25) (layer "F.Cu") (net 12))
 (segment (start 64.790004 71.582934) (end 64.790004 75.763715) (width 0.25) (layer "F.Cu") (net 12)))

